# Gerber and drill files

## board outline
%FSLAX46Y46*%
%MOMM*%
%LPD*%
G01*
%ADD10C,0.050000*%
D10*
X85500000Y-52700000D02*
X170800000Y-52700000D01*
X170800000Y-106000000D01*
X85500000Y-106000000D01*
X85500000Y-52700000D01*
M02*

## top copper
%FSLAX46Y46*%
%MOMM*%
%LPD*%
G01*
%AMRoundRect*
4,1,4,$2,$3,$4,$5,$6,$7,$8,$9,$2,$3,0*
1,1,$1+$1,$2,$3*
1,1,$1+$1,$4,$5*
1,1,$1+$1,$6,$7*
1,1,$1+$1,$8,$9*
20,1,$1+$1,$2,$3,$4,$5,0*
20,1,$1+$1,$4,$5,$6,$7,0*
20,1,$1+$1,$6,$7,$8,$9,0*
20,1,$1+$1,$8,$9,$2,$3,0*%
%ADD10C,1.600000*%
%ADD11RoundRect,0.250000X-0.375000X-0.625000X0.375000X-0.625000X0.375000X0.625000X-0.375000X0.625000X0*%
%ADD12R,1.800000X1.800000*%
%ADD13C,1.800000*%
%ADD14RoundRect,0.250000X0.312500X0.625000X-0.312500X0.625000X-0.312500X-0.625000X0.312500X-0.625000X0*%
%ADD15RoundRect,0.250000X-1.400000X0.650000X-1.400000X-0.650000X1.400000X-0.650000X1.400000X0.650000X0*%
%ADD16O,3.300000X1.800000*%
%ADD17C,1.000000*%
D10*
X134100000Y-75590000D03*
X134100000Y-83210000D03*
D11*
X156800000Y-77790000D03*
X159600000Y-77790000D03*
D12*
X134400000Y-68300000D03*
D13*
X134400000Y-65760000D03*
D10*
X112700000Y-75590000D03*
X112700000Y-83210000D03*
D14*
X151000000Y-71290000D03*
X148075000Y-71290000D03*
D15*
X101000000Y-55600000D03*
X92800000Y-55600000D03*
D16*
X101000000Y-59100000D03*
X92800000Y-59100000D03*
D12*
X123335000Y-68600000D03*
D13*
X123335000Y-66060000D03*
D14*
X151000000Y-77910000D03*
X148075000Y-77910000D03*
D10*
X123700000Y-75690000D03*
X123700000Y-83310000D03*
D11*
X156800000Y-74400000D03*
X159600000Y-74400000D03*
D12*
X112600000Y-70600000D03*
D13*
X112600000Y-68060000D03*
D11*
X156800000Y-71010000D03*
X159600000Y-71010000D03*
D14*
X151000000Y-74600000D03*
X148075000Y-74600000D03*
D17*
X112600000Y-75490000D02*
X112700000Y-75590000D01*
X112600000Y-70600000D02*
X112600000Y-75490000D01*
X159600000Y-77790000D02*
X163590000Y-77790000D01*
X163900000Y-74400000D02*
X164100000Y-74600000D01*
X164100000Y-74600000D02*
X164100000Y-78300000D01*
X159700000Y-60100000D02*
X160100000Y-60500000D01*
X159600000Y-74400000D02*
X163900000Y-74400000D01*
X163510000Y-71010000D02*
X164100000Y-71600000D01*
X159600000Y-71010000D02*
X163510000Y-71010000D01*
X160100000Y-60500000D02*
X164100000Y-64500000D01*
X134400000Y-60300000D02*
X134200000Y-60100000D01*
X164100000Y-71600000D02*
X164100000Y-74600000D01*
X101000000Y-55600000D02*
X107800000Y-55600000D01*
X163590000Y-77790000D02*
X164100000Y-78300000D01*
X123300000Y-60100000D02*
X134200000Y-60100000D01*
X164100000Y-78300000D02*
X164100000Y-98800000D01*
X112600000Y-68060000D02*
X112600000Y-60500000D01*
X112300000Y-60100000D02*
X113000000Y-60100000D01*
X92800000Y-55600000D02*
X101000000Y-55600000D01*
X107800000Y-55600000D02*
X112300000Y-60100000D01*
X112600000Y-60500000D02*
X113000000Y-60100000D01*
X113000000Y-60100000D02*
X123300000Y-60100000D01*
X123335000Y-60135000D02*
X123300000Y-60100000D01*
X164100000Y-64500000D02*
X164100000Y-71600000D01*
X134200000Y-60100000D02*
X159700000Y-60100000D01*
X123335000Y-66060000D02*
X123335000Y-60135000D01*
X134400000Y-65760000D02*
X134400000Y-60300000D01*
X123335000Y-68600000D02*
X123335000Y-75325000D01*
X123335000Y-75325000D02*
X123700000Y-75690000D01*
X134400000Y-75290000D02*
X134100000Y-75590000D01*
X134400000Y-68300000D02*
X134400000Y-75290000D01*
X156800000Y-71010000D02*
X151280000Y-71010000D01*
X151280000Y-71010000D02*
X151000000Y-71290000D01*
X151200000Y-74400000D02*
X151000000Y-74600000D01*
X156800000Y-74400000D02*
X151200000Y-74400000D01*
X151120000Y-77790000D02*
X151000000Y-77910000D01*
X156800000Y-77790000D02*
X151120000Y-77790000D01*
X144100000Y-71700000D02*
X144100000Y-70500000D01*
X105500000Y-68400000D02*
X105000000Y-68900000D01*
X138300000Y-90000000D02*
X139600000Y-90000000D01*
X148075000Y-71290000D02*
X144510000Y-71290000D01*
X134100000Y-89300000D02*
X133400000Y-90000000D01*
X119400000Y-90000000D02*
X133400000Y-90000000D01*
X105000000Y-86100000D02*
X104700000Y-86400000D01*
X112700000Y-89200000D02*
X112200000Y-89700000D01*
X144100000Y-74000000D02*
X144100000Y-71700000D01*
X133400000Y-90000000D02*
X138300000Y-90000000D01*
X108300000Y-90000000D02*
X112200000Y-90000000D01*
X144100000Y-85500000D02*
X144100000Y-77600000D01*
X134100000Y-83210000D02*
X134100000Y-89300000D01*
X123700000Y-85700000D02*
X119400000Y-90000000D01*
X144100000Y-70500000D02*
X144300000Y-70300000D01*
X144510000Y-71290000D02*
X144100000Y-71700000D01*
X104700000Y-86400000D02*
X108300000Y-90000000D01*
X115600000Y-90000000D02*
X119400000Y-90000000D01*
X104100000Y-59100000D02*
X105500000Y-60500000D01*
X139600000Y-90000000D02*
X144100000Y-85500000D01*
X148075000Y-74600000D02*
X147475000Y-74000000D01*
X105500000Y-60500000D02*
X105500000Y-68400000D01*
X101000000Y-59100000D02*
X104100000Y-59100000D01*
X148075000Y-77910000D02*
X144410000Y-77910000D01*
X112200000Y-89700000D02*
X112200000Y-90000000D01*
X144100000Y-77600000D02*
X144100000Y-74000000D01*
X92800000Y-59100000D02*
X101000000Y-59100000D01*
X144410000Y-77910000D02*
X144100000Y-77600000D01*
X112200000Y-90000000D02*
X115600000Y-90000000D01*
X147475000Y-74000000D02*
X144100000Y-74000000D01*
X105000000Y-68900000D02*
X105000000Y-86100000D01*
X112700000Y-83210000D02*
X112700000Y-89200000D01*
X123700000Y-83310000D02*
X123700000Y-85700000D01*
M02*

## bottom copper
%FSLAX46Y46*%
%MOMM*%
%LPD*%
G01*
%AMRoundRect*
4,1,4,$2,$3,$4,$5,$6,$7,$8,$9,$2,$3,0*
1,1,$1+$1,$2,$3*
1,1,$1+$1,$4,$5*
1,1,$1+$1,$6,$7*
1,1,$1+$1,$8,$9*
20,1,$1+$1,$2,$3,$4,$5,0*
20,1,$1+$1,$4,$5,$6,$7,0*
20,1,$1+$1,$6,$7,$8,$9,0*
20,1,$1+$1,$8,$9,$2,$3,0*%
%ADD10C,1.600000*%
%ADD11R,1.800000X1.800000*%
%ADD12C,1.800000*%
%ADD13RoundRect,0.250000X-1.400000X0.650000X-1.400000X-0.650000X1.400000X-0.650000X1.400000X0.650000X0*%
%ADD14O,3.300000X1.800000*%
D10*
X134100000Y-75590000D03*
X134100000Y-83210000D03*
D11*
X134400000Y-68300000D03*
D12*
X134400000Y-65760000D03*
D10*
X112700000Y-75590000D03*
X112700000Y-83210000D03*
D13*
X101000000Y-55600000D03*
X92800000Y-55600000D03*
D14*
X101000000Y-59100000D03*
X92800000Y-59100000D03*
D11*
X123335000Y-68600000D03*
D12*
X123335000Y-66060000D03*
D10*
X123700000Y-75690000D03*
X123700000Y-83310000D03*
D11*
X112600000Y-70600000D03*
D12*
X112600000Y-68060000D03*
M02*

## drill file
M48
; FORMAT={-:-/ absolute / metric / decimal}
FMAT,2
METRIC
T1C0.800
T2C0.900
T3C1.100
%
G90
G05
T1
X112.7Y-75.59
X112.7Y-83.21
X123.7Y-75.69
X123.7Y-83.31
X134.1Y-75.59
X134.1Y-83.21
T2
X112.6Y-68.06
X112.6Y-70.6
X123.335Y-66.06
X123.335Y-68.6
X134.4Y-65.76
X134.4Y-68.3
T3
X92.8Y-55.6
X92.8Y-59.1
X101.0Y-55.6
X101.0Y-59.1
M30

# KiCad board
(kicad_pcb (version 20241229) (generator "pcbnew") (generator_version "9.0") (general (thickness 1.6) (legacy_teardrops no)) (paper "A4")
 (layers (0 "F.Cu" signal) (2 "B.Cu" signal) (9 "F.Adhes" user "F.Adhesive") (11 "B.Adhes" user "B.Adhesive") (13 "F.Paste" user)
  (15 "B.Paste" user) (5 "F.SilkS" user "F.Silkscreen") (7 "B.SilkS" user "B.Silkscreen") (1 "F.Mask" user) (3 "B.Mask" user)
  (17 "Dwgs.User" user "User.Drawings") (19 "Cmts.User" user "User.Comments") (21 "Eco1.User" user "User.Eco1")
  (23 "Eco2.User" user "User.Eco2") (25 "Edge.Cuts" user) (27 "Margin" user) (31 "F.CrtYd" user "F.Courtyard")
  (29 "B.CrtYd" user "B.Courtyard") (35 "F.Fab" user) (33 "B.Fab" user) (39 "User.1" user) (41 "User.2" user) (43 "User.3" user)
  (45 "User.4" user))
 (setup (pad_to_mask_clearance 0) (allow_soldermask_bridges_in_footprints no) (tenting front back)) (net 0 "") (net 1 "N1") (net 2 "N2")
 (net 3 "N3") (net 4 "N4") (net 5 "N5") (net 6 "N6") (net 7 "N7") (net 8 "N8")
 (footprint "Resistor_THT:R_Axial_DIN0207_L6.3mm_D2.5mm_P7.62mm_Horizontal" (layer "F.Cu") (at 134.1 75.59 -90)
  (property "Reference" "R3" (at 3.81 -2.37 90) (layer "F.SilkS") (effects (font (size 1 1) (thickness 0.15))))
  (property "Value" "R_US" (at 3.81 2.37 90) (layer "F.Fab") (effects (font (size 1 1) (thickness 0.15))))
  (pad "1" thru_hole circle (at 0 0 270) (size 1.6 1.6) (drill 0.8) (layers "*.Cu" "*.Mask") (remove_unused_layers no) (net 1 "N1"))
  (pad "2" thru_hole circle (at 7.62 0 270) (size 1.6 1.6) (drill 0.8) (layers "*.Cu" "*.Mask") (remove_unused_layers no) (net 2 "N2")))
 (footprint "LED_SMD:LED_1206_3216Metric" (layer "F.Cu") (at 158.2 77.79)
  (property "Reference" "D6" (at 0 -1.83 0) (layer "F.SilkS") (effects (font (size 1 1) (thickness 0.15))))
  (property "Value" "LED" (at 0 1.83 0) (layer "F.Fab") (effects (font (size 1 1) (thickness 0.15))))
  (pad "1" smd roundrect (at -1.4 0) (size 1.25 1.75) (layers "F.Cu" "F.Mask" "F.Paste") (roundrect_rratio 0.2) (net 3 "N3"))
  (pad "2" smd roundrect (at 1.4 0) (size 1.25 1.75) (layers "F.Cu" "F.Mask" "F.Paste") (roundrect_rratio 0.2) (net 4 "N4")))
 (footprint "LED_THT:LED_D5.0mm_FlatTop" (layer "F.Cu") (at 134.4 68.3 90)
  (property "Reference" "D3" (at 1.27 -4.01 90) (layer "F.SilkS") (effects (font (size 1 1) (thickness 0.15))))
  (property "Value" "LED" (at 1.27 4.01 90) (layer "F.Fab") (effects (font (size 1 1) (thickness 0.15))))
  (pad "1" thru_hole rect (at 0 0 90) (size 1.8 1.8) (drill 0.9) (layers "*.Cu" "*.Mask") (remove_unused_layers no) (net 1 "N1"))
  (pad "2" thru_hole circle (at 2.54 0 90) (size 1.8 1.8) (drill 0.9) (layers "*.Cu" "*.Mask") (remove_unused_layers no) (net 4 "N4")))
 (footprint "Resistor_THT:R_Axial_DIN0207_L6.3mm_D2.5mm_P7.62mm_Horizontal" (layer "F.Cu") (at 112.7 75.59 -90)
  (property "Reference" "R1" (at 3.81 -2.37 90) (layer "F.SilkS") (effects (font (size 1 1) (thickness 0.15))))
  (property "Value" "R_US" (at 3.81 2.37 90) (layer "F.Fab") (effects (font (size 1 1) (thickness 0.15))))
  (pad "1" thru_hole circle (at 0 0 270) (size 1.6 1.6) (drill 0.8) (layers "*.Cu" "*.Mask") (remove_unused_layers no) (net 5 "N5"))
  (pad "2" thru_hole circle (at 7.62 0 270) (size 1.6 1.6) (drill 0.8) (layers "*.Cu" "*.Mask") (remove_unused_layers no) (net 2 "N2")))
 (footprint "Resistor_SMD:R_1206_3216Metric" (layer "F.Cu") (at 149.5375 71.29 180)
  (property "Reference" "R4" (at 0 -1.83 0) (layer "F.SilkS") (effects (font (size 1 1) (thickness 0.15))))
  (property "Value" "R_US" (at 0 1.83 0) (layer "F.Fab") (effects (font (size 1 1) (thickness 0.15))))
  (pad "1" smd roundrect (at -1.4625 0 180) (size 1.125 1.75) (layers "F.Cu" "F.Mask" "F.Paste") (roundrect_rratio 0.222222) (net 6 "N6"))
  (pad "2" smd roundrect (at 1.4625 0 180) (size 1.125 1.75) (layers "F.Cu" "F.Mask" "F.Paste") (roundrect_rratio 0.222222) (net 2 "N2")))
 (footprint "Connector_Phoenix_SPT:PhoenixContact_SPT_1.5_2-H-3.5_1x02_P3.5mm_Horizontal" (layer "F.Cu") (at 101 55.6 -90)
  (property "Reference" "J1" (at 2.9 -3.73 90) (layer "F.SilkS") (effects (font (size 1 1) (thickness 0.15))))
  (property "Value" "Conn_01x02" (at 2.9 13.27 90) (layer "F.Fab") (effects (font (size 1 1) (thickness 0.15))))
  (pad "1" thru_hole roundrect (at 0 0 270) (size 1.8 3.3) (drill 1.1) (layers "*.Cu" "*.Mask") (remove_unused_layers no)
   (roundrect_rratio 0.138889) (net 4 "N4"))
  (pad "1" thru_hole roundrect (at 0 8.2 270) (size 1.8 3.3) (drill 1.1) (layers "*.Cu" "*.Mask") (remove_unused_layers no)
   (roundrect_rratio 0.138889) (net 4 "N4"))
  (pad "2" thru_hole oval (at 3.5 0 270) (size 1.8 3.3) (drill 1.1) (layers "*.Cu" "*.Mask") (remove_unused_layers no) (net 2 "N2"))
  (pad "2" thru_hole oval (at 3.5 8.2 270) (size 1.8 3.3) (drill 1.1) (layers "*.Cu" "*.Mask") (remove_unused_layers no) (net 2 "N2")))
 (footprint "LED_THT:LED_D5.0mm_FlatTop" (layer "F.Cu") (at 123.335 68.6 90)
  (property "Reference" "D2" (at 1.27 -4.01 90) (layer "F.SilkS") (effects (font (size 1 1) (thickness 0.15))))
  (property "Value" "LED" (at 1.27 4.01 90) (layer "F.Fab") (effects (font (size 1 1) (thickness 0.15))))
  (pad "1" thru_hole rect (at 0 0 90) (size 1.8 1.8) (drill 0.9) (layers "*.Cu" "*.Mask") (remove_unused_layers no) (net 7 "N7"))
  (pad "2" thru_hole circle (at 2.54 0 90) (size 1.8 1.8) (drill 0.9) (layers "*.Cu" "*.Mask") (remove_unused_layers no) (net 4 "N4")))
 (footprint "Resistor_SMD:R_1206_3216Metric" (layer "F.Cu") (at 149.5375 77.91 180)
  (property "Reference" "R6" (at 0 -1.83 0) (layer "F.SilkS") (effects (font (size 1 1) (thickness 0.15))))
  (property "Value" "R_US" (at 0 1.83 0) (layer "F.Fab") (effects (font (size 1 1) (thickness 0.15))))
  (pad "1" smd roundrect (at -1.4625 0 180) (size 1.125 1.75) (layers "F.Cu" "F.Mask" "F.Paste") (roundrect_rratio 0.222222) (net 3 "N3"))
  (pad "2" smd roundrect (at 1.4625 0 180) (size 1.125 1.75) (layers "F.Cu" "F.Mask" "F.Paste") (roundrect_rratio 0.222222) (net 2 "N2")))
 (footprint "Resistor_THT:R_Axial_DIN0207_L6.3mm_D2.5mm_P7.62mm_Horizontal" (layer "F.Cu") (at 123.7 75.69 -90)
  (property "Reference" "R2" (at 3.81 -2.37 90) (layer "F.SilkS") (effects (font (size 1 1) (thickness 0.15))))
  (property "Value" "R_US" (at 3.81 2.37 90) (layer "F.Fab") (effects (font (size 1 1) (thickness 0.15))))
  (pad "1" thru_hole circle (at 0 0 270) (size 1.6 1.6) (drill 0.8) (layers "*.Cu" "*.Mask") (remove_unused_layers no) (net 7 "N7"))
  (pad "2" thru_hole circle (at 7.62 0 270) (size 1.6 1.6) (drill 0.8) (layers "*.Cu" "*.Mask") (remove_unused_layers no) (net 2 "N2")))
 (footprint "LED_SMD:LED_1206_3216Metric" (layer "F.Cu") (at 158.2 74.4)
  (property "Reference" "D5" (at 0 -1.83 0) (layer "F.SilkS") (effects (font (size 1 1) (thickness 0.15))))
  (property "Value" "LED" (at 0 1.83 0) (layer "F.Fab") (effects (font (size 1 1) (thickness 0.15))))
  (pad "1" smd roundrect (at -1.4 0) (size 1.25 1.75) (layers "F.Cu" "F.Mask" "F.Paste") (roundrect_rratio 0.2) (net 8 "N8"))
  (pad "2" smd roundrect (at 1.4 0) (size 1.25 1.75) (layers "F.Cu" "F.Mask" "F.Paste") (roundrect_rratio 0.2) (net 4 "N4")))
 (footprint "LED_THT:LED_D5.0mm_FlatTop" (layer "F.Cu") (at 112.6 70.6 90)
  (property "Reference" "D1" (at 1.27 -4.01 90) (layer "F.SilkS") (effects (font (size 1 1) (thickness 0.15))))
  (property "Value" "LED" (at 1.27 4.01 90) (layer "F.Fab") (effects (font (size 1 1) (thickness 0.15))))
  (pad "1" thru_hole rect (at 0 0 90) (size 1.8 1.8) (drill 0.9) (layers "*.Cu" "*.Mask") (remove_unused_layers no) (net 5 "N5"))
  (pad "2" thru_hole circle (at 2.54 0 90) (size 1.8 1.8) (drill 0.9) (layers "*.Cu" "*.Mask") (remove_unused_layers no) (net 4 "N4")))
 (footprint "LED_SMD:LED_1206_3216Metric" (layer "F.Cu") (at 158.2 71.01)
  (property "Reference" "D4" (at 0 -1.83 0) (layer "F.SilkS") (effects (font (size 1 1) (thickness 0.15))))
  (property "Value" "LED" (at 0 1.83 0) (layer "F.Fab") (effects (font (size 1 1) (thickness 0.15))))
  (pad "1" smd roundrect (at -1.4 0) (size 1.25 1.75) (layers "F.Cu" "F.Mask" "F.Paste") (roundrect_rratio 0.2) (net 6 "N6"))
  (pad "2" smd roundrect (at 1.4 0) (size 1.25 1.75) (layers "F.Cu" "F.Mask" "F.Paste") (roundrect_rratio 0.2) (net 4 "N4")))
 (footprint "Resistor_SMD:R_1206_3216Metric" (layer "F.Cu") (at 149.5375 74.6 180)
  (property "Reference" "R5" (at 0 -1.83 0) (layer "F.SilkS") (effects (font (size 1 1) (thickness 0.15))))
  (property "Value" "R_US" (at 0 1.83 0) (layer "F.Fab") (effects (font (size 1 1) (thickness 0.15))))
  (pad "1" smd roundrect (at -1.4625 0 180) (size 1.125 1.75) (layers "F.Cu" "F.Mask" "F.Paste") (roundrect_rratio 0.222222) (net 8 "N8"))
  (pad "2" smd roundrect (at 1.4625 0 180) (size 1.125 1.75) (layers "F.Cu" "F.Mask" "F.Paste") (roundrect_rratio 0.222222) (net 2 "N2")))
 (gr_rect (start 85.5 52.7) (end 170.8 106) (stroke (width 0.05) (type default)) (fill no) (layer "Edge.Cuts"))
 (segment (start 112.6 75.49) (end 112.7 75.59) (width 1) (layer "F.Cu") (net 5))
 (segment (start 112.6 70.6) (end 112.6 75.49) (width 1) (layer "F.Cu") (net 5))
 (segment (start 159.6 77.79) (end 163.59 77.79) (width 1) (layer "F.Cu") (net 4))
 (segment (start 163.9 74.4) (end 164.1 74.6) (width 1) (layer "F.Cu") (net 4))
 (segment (start 164.1 74.6) (end 164.1 78.3) (width 1) (layer "F.Cu") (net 4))
 (segment (start 159.7 60.1) (end 160.1 60.5) (width 1) (layer "F.Cu") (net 4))
 (segment (start 159.6 74.4) (end 163.9 74.4) (width 1) (layer "F.Cu") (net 4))
 (segment (start 163.51 71.01) (end 164.1 71.6) (width 1) (layer "F.Cu") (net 4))
 (segment (start 159.6 71.01) (end 163.51 71.01) (width 1) (layer "F.Cu") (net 4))
 (segment (start 160.1 60.5) (end 164.1 64.5) (width 1) (layer "F.Cu") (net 4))
 (segment (start 134.4 60.3) (end 134.2 60.1) (width 1) (layer "F.Cu") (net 4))
 (segment (start 164.1 71.6) (end 164.1 74.6) (width 1) (layer "F.Cu") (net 4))
 (segment (start 101 55.6) (end 107.8 55.6) (width 1) (layer "F.Cu") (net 4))
 (segment (start 163.59 77.79) (end 164.1 78.3) (width 1) (layer "F.Cu") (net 4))
 (segment (start 123.3 60.1) (end 134.2 60.1) (width 1) (layer "F.Cu") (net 4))
 (segment (start 164.1 78.3) (end 164.1 98.8) (width 1) (layer "F.Cu") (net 4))
 (segment (start 112.6 68.06) (end 112.6 60.5) (width 1) (layer "F.Cu") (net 4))
 (segment (start 112.3 60.1) (end 113 60.1) (width 1) (layer "F.Cu") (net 4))
 (segment (start 92.8 55.6) (end 101 55.6) (width 1) (layer "F.Cu") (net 4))
 (segment (start 107.8 55.6) (end 112.3 60.1) (width 1) (layer "F.Cu") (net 4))
 (segment (start 112.6 60.5) (end 113 60.1) (width 1) (layer "F.Cu") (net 4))
 (segment (start 113 60.1) (end 123.3 60.1) (width 1) (layer "F.Cu") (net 4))
 (segment (start 123.335 60.135) (end 123.3 60.1) (width 1) (layer "F.Cu") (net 4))
 (segment (start 164.1 64.5) (end 164.1 71.6) (width 1) (layer "F.Cu") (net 4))
 (segment (start 134.2 60.1) (end 159.7 60.1) (width 1) (layer "F.Cu") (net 4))
 (segment (start 123.335 66.06) (end 123.335 60.135) (width 1) (layer "F.Cu") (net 4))
 (segment (start 134.4 65.76) (end 134.4 60.3) (width 1) (layer "F.Cu") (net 4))
 (segment (start 123.335 68.6) (end 123.335 75.325) (width 1) (layer "F.Cu") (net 7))
 (segment (start 123.335 75.325) (end 123.7 75.69) (width 1) (layer "F.Cu") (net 7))
 (segment (start 134.4 75.29) (end 134.1 75.59) (width 1) (layer "F.Cu") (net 1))
 (segment (start 134.4 68.3) (end 134.4 75.29) (width 1) (layer "F.Cu") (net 1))
 (segment (start 156.8 71.01) (end 151.28 71.01) (width 1) (layer "F.Cu") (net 6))
 (segment (start 151.28 71.01) (end 151 71.29) (width 1) (layer "F.Cu") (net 6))
 (segment (start 151.2 74.4) (end 151 74.6) (width 1) (layer "F.Cu") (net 8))
 (segment (start 156.8 74.4) (end 151.2 74.4) (width 1) (layer "F.Cu") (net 8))
 (segment (start 151.12 77.79) (end 151 77.91) (width 1) (layer "F.Cu") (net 3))
 (segment (start 156.8 77.79) (end 151.12 77.79) (width 1) (layer "F.Cu") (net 3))
 (segment (start 144.1 71.7) (end 144.1 70.5) (width 1) (layer "F.Cu") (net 2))
 (segment (start 105.5 68.4) (end 105 68.9) (width 1) (layer "F.Cu") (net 2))
 (segment (start 138.3 90) (end 139.6 90) (width 1) (layer "F.Cu") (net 2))
 (segment (start 148.075 71.29) (end 144.51 71.29) (width 1) (layer "F.Cu") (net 2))
 (segment (start 134.1 89.3) (end 133.4 90) (width 1) (layer "F.Cu") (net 2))
 (segment (start 119.4 90) (end 133.4 90) (width 1) (layer "F.Cu") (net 2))
 (segment (start 105 86.1) (end 104.7 86.4) (width 1) (layer "F.Cu") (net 2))
 (segment (start 112.7 89.2) (end 112.2 89.7) (width 1) (layer "F.Cu") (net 2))
 (segment (start 144.1 74) (end 144.1 71.7) (width 1) (layer "F.Cu") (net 2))
 (segment (start 133.4 90) (end 138.3 90) (width 1) (layer "F.Cu") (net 2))
 (segment (start 108.3 90) (end 112.2 90) (width 1) (layer "F.Cu") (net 2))
 (segment (start 144.1 85.5) (end 144.1 77.6) (width 1) (layer "F.Cu") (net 2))
 (segment (start 134.1 83.21) (end 134.1 89.3) (width 1) (layer "F.Cu") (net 2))
 (segment (start 123.7 85.7) (end 119.4 90) (width 1) (layer "F.Cu") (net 2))
 (segment (start 144.1 70.5) (end 144.3 70.3) (width 1) (layer "F.Cu") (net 2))
 (segment (start 144.51 71.29) (end 144.1 71.7) (width 1) (layer "F.Cu") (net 2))
 (segment (start 104.7 86.4) (end 108.3 90) (width 1) (layer "F.Cu") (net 2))
 (segment (start 115.6 90) (end 119.4 90) (width 1) (layer "F.Cu") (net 2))
 (segment (start 104.1 59.1) (end 105.5 60.5) (width 1) (layer "F.Cu") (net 2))
 (segment (start 139.6 90) (end 144.1 85.5) (width 1) (layer "F.Cu") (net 2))
 (segment (start 148.075 74.6) (end 147.475 74) (width 1) (layer "F.Cu") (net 2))
 (segment (start 105.5 60.5) (end 105.5 68.4) (width 1) (layer "F.Cu") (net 2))
 (segment (start 101 59.1) (end 104.1 59.1) (width 1) (layer "F.Cu") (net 2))
 (segment (start 148.075 77.91) (end 144.41 77.91) (width 1) (layer "F.Cu") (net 2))
 (segment (start 112.2 89.7) (end 112.2 90) (width 1) (layer "F.Cu") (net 2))
 (segment (start 144.1 77.6) (end 144.1 74) (width 1) (layer "F.Cu") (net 2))
 (segment (start 92.8 59.1) (end 101 59.1) (width 1) (layer "F.Cu") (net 2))
 (segment (start 144.41 77.91) (end 144.1 77.6) (width 1) (layer "F.Cu") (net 2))
 (segment (start 112.2 90) (end 115.6 90) (width 1) (layer "F.Cu") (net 2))
 (segment (start 147.475 74) (end 144.1 74) (width 1) (layer "F.Cu") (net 2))
 (segment (start 105 68.9) (end 105 86.1) (width 1) (layer "F.Cu") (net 2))
 (segment (start 112.7 83.21) (end 112.7 89.2) (width 1) (layer "F.Cu") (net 2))
 (segment (start 123.7 83.31) (end 123.7 85.7) (width 1) (layer "F.Cu") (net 2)))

